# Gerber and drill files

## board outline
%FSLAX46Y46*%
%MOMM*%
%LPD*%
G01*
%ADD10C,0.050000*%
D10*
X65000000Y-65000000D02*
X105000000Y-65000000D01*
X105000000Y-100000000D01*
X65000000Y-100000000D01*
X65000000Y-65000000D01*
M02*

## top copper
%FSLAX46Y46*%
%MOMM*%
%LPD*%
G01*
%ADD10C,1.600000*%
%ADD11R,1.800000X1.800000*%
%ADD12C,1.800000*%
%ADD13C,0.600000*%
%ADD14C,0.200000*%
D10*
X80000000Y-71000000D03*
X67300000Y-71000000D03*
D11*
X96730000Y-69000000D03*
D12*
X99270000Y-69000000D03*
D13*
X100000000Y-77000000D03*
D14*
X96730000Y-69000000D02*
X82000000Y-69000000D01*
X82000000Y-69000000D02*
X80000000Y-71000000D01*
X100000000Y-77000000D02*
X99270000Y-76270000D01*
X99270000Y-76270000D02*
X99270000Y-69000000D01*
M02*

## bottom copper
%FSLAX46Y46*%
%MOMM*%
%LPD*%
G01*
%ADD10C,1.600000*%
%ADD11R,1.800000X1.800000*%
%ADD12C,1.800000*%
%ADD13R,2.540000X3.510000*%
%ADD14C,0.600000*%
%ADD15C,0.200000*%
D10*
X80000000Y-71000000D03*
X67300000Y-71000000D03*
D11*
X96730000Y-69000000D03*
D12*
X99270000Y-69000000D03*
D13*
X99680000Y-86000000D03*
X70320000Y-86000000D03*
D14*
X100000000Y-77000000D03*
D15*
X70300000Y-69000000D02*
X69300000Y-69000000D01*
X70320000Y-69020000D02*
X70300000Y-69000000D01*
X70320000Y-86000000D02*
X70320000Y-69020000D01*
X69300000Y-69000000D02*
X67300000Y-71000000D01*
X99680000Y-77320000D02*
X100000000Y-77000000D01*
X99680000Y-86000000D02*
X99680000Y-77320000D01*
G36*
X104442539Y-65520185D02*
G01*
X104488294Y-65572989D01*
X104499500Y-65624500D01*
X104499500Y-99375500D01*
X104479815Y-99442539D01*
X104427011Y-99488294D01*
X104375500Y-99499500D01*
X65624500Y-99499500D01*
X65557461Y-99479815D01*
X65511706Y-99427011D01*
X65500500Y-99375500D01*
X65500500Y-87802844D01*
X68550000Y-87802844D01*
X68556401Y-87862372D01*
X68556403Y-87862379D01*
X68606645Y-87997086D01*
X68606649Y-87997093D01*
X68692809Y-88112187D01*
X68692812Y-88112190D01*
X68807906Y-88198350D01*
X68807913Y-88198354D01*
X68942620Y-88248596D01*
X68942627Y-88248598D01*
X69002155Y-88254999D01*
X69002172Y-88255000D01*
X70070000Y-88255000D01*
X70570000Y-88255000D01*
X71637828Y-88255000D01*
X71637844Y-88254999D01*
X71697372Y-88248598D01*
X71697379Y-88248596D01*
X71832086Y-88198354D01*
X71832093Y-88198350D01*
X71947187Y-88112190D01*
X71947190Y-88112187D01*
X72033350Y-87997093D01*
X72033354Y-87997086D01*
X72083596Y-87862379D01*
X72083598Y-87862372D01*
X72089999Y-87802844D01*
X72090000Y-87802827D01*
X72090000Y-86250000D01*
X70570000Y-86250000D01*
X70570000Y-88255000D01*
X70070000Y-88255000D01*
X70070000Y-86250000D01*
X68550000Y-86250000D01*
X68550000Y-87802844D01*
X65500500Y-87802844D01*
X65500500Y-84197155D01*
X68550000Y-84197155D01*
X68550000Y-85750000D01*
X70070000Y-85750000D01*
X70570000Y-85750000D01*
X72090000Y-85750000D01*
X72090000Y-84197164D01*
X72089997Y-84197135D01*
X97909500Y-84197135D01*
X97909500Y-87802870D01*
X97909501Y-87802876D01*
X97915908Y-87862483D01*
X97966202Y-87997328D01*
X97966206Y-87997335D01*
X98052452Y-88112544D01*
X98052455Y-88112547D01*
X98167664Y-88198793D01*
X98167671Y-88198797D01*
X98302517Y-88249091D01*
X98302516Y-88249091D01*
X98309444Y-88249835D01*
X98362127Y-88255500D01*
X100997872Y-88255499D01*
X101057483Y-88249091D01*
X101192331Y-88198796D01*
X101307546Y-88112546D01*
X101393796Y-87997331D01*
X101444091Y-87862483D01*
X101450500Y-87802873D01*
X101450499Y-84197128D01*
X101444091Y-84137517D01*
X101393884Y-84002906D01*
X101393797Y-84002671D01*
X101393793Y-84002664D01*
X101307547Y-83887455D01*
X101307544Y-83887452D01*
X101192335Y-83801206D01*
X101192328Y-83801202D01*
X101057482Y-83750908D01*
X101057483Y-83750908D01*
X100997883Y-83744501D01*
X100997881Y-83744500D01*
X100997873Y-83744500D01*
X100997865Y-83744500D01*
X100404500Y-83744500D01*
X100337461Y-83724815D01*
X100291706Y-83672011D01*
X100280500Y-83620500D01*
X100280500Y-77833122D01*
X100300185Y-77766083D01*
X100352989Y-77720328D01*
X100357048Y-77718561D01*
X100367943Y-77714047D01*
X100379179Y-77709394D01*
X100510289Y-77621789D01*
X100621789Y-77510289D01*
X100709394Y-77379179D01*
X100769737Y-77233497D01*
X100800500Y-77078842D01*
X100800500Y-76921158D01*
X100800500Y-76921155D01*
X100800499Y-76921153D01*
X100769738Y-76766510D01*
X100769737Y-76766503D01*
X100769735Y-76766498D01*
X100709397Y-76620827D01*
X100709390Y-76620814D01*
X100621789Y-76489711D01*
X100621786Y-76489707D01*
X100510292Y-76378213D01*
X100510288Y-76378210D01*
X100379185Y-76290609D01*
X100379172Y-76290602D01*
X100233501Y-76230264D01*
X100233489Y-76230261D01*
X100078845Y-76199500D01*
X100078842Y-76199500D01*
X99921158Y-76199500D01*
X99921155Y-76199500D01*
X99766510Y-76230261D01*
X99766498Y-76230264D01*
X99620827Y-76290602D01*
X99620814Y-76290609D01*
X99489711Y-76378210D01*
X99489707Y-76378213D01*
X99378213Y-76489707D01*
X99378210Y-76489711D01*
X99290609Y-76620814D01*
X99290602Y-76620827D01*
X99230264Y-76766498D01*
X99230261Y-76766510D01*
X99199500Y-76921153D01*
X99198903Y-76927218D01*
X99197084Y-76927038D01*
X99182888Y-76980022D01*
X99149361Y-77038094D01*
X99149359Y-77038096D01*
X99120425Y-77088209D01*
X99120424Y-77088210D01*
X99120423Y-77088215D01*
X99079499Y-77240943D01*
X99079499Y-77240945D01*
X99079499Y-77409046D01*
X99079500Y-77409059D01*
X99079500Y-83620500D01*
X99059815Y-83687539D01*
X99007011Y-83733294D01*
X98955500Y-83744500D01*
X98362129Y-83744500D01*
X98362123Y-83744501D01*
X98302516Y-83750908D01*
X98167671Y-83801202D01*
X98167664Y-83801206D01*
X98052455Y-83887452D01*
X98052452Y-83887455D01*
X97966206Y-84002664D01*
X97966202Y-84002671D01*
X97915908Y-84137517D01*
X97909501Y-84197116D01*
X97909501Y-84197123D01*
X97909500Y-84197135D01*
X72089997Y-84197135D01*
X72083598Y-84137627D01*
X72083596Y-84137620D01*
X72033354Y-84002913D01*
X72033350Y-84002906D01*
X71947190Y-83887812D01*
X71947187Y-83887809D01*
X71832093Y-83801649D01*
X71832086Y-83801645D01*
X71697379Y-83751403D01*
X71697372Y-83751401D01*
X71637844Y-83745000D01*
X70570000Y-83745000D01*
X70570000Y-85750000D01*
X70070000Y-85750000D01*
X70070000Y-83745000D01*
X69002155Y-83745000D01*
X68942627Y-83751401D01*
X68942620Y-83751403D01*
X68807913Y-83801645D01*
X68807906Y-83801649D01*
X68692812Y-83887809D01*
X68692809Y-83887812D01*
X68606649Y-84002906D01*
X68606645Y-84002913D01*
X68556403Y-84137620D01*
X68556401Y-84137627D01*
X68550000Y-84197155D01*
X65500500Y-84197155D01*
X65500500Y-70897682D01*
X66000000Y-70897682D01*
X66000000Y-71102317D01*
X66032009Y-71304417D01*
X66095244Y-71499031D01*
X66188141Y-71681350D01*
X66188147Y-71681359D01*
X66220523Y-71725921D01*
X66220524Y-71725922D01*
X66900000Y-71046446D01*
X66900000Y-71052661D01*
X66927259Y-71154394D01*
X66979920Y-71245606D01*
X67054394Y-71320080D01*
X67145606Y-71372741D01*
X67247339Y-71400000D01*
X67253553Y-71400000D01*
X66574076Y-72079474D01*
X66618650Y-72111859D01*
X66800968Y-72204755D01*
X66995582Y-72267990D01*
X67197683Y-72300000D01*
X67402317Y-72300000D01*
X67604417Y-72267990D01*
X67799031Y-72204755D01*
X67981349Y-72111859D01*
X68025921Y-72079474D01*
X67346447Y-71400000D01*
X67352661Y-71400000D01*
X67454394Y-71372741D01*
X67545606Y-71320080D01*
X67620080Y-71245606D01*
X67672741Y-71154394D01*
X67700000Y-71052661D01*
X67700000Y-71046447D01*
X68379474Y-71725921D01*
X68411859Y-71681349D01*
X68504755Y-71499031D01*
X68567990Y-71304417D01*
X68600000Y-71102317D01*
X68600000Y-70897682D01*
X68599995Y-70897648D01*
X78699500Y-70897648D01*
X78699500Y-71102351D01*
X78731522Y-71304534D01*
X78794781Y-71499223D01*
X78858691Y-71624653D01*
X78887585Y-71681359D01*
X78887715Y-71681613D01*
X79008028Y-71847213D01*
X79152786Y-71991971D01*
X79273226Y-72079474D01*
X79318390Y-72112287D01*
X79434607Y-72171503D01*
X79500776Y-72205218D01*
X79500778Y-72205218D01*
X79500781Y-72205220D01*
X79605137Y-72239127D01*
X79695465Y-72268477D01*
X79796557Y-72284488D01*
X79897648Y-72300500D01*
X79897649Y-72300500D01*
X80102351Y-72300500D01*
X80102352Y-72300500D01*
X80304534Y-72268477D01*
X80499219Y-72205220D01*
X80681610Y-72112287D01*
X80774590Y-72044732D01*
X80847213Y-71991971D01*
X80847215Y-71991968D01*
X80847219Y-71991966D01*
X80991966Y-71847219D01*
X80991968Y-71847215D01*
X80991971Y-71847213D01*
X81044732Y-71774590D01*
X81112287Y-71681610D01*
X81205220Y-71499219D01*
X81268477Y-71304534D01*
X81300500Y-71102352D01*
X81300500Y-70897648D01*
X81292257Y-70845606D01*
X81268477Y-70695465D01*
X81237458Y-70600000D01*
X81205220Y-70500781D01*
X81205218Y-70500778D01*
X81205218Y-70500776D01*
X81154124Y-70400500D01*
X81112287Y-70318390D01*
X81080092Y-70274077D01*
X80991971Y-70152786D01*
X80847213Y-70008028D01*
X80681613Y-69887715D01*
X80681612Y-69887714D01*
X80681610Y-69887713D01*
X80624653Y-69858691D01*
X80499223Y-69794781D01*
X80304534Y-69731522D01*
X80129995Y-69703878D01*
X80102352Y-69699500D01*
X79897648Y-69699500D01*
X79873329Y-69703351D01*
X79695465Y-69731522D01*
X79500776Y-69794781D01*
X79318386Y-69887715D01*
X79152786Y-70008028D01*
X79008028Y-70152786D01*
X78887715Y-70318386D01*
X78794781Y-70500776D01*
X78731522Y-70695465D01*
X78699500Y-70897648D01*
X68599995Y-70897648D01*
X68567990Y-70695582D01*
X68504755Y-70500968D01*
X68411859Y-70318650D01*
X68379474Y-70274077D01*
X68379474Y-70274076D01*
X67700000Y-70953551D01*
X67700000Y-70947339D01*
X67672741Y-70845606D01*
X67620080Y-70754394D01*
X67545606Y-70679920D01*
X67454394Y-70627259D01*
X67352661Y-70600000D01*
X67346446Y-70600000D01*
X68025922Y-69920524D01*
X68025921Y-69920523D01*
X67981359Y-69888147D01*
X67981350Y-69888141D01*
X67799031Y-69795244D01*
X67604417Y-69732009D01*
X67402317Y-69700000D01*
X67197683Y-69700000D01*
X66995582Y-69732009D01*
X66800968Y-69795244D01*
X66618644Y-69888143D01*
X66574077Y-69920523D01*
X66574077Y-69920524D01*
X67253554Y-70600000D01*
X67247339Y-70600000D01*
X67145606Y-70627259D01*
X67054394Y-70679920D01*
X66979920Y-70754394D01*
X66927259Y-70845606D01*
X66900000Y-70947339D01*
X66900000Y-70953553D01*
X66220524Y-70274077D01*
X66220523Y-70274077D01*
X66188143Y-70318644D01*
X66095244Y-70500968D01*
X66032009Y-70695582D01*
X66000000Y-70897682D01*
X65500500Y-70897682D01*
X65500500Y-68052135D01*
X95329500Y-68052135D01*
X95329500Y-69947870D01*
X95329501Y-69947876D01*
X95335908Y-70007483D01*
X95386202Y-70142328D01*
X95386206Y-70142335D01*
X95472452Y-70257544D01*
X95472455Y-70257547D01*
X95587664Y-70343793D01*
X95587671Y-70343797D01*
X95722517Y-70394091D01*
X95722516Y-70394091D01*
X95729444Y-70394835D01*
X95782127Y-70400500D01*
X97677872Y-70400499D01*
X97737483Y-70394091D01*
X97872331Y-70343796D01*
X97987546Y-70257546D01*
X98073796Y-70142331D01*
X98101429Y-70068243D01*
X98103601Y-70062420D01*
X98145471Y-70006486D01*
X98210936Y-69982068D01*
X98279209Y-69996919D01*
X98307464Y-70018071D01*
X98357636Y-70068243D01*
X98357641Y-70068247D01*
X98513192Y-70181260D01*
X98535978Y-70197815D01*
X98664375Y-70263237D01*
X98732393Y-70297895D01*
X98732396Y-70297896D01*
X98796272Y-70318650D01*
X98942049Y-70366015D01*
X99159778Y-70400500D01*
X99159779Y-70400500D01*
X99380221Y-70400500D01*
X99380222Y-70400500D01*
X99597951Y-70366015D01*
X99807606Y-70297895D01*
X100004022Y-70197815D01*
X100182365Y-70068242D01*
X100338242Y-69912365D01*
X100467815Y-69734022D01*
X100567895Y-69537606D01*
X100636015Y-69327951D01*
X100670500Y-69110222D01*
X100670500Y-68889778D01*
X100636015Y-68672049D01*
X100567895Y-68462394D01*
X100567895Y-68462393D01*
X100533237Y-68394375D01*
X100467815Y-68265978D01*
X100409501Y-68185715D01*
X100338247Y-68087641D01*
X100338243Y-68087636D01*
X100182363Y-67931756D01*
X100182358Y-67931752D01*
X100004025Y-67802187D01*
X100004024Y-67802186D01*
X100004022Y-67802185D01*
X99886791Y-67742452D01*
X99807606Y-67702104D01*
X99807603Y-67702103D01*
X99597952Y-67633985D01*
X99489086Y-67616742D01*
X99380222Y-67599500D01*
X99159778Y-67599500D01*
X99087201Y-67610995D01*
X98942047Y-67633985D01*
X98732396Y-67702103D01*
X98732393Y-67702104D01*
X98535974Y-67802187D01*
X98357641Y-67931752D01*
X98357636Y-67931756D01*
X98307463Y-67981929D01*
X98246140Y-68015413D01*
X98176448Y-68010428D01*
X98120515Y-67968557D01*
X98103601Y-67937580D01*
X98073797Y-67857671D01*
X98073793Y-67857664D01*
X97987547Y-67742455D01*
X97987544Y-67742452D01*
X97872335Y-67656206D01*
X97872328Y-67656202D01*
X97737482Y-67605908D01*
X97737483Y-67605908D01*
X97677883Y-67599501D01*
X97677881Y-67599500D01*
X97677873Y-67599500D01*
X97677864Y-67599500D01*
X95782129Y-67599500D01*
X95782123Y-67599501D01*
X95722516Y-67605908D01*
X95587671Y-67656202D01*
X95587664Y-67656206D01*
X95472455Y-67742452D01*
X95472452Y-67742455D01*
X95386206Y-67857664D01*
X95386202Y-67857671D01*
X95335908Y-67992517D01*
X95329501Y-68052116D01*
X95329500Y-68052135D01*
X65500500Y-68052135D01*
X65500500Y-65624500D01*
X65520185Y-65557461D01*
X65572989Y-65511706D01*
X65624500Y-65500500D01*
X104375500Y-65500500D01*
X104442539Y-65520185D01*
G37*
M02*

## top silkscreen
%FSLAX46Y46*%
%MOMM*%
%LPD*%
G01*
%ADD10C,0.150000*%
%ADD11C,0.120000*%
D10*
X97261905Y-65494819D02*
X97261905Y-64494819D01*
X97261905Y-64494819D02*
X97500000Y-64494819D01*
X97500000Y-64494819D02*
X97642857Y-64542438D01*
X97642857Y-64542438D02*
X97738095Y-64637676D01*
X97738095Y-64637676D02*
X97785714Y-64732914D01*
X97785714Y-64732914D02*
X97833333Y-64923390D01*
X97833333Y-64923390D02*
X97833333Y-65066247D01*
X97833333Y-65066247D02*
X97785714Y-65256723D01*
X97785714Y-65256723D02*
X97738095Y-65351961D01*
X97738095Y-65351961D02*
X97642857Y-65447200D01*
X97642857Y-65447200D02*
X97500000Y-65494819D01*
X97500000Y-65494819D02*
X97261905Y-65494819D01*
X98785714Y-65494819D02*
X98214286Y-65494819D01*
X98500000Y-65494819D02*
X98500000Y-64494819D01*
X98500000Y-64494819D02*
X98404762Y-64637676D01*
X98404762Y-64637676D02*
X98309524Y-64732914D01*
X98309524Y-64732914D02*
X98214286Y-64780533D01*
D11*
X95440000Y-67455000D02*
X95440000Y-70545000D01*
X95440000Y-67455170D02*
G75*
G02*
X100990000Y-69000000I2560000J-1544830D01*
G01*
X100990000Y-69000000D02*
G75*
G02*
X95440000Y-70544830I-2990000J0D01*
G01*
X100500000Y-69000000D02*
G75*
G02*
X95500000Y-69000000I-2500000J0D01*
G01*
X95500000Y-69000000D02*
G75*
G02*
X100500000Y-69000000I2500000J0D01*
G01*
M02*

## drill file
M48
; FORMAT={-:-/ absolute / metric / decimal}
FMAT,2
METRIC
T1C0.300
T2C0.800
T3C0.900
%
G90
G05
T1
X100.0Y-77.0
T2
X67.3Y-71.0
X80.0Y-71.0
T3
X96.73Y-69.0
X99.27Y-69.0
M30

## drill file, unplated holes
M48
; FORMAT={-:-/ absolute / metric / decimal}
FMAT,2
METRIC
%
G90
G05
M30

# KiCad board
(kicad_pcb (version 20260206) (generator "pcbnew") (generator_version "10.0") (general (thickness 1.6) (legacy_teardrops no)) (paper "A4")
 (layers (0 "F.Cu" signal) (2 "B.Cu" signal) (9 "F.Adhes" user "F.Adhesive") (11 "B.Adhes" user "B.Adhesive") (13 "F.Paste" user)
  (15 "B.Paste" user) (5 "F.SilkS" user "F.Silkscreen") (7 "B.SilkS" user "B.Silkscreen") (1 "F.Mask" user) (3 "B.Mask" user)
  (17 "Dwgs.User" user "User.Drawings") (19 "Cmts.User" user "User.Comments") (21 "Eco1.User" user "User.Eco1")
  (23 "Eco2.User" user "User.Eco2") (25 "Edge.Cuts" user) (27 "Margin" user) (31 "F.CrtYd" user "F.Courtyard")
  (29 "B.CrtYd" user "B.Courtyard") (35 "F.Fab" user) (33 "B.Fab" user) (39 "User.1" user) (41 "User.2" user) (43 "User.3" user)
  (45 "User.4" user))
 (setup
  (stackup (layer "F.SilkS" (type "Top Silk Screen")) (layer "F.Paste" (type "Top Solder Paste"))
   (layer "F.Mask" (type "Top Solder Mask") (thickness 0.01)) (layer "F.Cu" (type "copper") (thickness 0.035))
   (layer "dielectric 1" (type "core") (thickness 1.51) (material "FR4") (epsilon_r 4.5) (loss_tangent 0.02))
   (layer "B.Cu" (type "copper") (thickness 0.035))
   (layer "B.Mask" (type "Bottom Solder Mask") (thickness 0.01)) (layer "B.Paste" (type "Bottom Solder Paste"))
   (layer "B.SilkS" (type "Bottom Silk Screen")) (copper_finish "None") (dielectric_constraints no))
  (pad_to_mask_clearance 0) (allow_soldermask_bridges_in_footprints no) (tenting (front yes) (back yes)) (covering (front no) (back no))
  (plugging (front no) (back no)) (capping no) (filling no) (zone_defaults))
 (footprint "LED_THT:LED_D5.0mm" (layer "F.Cu") (at 96.73 69)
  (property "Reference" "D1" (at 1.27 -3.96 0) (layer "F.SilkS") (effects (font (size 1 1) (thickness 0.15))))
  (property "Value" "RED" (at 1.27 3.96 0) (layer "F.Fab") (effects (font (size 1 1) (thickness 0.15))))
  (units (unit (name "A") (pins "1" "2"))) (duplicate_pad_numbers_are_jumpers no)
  (fp_line (start -1.29 -1.545) (end -1.29 1.545) (stroke (width 0.12) (type solid)) (layer "F.SilkS"))
  (fp_arc (start -1.29 -1.54483) (mid 2.071779 -2.880495) (end 4.26 0) (stroke (width 0.12) (type solid)) (layer "F.SilkS"))
  (fp_arc (start 4.26 0) (mid 2.071779 2.880495) (end -1.29 1.54483) (stroke (width 0.12) (type solid)) (layer "F.SilkS"))
  (fp_circle (center 1.27 0) (end 3.77 0) (stroke (width 0.12) (type solid)) (fill no) (layer "F.SilkS"))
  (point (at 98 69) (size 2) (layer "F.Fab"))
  (pad "1" thru_hole rect (at 0 0) (size 1.8 1.8) (drill 0.9) (layers "*.Cu" "*.Mask") (remove_unused_layers no) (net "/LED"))
  (pad "2" thru_hole circle (at 2.54 0) (size 1.8 1.8) (drill 0.9) (layers "*.Cu" "*.Mask") (remove_unused_layers no) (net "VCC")))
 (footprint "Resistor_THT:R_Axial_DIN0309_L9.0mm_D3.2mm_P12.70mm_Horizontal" (layer "B.Cu") (at 80 71 180)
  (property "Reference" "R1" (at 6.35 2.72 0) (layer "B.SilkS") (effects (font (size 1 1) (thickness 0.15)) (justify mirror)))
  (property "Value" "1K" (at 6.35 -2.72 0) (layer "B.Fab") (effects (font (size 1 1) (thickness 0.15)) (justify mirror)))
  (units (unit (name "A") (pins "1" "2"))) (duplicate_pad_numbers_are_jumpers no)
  (pad "1" thru_hole circle (at 0 0 180) (size 1.6 1.6) (drill 0.8) (layers "*.Cu" "*.Mask") (remove_unused_layers no) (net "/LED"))
  (pad "2" thru_hole circle (at 12.7 0 180) (size 1.6 1.6) (drill 0.8) (layers "*.Cu" "*.Mask") (remove_unused_layers no) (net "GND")))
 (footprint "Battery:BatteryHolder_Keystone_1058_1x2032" (layer "B.Cu") (at 85 86 180)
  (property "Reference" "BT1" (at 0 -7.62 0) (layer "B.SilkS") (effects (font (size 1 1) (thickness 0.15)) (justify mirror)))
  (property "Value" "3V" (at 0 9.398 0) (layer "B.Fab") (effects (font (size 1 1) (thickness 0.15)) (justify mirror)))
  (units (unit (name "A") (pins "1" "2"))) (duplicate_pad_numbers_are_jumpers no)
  (pad "1" smd rect (at -14.68 0 180) (size 2.54 3.51) (layers "B.Cu" "B.Mask" "B.Paste") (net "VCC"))
  (pad "2" smd rect (at 14.68 0 180) (size 2.54 3.51) (layers "B.Cu" "B.Mask" "B.Paste") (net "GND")))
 (gr_rect (start 65 65) (end 105 100) (stroke (width 0.05) (type default)) (fill no) (layer "Edge.Cuts"))
 (segment (start 70.3 69) (end 69.3 69) (width 0.2) (layer "B.Cu") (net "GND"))
 (segment (start 70.32 86) (end 70.32 69.02) (width 0.2) (layer "B.Cu") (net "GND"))
 (segment (start 69.3 69) (end 67.3 71) (width 0.2) (layer "B.Cu") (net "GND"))
 (segment (start 70.32 69.02) (end 70.3 69) (width 0.2) (layer "B.Cu") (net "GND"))
 (segment (start 100 77) (end 99.27 76.27) (width 0.2) (layer "F.Cu") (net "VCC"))
 (segment (start 99.27 76.27) (end 99.27 69) (width 0.2) (layer "F.Cu") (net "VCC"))
 (via (at 100 77) (size 0.6) (drill 0.3) (layers "F.Cu" "B.Cu") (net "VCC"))
 (segment (start 99.68 86) (end 99.68 77.32) (width 0.2) (layer "B.Cu") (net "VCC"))
 (segment (start 99.68 77.32) (end 100 77) (width 0.2) (layer "B.Cu") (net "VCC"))
 (segment (start 82 69) (end 80 71) (width 0.2) (layer "F.Cu") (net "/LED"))
 (segment (start 96.73 69) (end 82 69) (width 0.2) (layer "F.Cu") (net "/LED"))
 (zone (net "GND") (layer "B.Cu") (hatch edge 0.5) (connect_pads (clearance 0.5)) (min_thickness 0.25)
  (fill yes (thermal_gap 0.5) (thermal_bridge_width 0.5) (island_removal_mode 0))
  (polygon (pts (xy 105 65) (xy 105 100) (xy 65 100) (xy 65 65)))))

